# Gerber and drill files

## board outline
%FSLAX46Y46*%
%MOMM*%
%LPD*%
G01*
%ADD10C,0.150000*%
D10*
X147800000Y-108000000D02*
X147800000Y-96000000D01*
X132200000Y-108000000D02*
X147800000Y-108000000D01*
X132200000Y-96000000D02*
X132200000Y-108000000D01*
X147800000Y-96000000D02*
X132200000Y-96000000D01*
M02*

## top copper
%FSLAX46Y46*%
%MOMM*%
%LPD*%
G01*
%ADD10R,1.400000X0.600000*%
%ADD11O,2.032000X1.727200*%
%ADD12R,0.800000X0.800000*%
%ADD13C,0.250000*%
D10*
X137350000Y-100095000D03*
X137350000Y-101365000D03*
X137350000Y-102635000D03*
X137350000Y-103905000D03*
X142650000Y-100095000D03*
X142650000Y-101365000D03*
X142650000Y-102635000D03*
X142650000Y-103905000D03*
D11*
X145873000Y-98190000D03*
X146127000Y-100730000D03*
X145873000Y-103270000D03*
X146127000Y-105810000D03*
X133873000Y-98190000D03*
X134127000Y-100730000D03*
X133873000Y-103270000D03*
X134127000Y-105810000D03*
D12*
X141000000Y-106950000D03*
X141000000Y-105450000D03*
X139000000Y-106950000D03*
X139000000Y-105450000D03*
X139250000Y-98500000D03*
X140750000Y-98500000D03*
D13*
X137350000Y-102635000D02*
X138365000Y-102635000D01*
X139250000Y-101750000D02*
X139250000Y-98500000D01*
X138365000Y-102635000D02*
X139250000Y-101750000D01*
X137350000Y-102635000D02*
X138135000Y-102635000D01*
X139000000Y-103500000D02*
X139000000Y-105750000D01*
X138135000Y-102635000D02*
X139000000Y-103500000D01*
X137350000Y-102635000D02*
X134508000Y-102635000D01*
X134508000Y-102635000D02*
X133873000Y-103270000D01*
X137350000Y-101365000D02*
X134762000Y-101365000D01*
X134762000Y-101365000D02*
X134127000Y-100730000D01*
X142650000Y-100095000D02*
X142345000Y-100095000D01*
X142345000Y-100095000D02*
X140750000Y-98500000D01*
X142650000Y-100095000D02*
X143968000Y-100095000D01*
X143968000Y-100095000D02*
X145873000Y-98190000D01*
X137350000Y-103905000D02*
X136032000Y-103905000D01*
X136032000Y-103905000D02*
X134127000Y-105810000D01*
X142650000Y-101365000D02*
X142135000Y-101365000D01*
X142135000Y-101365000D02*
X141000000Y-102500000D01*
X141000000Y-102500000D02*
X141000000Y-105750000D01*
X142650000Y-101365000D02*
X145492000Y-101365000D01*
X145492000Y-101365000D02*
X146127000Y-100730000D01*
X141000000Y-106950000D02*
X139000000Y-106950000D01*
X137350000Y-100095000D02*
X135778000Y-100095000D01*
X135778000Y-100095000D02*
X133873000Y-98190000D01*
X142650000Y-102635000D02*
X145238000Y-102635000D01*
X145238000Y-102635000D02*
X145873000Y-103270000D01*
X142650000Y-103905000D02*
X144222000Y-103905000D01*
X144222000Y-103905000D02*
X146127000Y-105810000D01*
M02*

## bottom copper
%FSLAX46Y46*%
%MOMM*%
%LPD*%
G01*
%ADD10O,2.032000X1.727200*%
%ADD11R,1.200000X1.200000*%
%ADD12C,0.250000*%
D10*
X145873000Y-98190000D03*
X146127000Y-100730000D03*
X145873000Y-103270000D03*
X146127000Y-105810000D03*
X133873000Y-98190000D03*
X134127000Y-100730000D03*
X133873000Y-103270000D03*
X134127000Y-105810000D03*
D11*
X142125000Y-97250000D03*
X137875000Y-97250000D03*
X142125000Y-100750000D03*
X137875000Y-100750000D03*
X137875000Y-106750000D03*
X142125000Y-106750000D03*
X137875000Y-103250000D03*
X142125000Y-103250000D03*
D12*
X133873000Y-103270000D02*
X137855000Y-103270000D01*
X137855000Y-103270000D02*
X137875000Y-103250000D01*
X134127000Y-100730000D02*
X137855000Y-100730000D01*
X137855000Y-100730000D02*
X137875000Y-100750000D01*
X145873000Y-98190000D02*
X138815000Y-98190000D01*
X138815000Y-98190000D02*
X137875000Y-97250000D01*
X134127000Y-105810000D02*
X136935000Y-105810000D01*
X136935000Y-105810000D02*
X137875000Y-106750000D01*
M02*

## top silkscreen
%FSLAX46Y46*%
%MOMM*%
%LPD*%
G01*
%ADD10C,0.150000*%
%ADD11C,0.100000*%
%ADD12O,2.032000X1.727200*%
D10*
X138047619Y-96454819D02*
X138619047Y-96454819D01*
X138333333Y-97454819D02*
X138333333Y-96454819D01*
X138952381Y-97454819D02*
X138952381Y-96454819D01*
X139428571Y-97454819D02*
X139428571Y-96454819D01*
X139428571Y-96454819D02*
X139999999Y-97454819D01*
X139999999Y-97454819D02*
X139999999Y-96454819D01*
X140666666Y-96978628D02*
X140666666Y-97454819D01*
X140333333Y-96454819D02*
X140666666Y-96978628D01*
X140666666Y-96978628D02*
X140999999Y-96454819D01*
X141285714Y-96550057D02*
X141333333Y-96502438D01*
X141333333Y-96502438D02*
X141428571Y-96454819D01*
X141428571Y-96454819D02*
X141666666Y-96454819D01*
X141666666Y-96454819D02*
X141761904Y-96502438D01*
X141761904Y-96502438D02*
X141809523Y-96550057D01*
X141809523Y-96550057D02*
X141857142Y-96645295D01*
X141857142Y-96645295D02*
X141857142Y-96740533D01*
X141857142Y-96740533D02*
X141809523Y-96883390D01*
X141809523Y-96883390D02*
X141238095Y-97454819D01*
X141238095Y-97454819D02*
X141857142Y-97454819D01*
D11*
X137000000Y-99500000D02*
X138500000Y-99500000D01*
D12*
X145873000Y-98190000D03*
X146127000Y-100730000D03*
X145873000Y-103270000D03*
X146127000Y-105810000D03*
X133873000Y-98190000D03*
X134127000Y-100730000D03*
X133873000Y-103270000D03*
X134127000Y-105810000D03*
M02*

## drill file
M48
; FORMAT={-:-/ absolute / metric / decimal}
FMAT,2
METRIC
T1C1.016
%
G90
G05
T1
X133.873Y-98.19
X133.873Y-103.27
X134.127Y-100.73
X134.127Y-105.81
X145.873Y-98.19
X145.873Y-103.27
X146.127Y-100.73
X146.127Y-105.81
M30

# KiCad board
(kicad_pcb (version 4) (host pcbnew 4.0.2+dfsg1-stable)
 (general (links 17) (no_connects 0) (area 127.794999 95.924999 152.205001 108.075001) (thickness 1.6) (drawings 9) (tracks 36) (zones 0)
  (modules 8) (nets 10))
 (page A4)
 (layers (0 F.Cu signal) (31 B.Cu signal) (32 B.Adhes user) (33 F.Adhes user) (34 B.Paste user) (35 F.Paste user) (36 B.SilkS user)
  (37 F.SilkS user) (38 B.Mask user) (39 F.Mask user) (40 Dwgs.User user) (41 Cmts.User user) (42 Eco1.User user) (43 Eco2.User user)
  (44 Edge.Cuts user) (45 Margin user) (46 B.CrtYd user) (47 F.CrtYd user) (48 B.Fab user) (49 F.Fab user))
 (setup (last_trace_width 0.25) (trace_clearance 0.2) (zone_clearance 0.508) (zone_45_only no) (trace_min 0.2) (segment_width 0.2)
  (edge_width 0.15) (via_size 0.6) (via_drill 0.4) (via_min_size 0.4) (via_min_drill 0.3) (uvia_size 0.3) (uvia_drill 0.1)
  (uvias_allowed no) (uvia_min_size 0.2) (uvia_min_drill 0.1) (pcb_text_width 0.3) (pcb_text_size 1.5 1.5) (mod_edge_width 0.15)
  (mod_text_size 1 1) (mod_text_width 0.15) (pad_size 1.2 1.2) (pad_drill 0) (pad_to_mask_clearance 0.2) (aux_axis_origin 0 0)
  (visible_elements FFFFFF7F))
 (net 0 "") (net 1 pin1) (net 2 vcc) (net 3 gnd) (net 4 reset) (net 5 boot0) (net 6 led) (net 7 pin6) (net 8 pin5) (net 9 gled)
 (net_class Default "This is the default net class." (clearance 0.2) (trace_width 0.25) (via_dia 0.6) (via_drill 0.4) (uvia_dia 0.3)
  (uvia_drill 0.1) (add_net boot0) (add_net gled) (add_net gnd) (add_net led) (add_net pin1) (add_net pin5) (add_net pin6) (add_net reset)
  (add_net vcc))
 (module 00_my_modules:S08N (layer F.Cu) (at 140 102)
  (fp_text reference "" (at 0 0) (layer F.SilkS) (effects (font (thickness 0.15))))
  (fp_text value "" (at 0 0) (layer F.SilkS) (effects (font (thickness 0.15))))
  (fp_line (start -3 -2.5) (end -1.5 -2.5) (layer F.SilkS) (width 0.1))
  (pad 1 smd rect (at -2.65 -1.905) (size 1.4 0.6) (layers F.Cu F.Paste F.Mask) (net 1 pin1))
  (pad VCC smd rect (at -2.65 -0.635) (size 1.4 0.6) (layers F.Cu F.Paste F.Mask) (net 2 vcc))
  (pad GND smd rect (at -2.65 0.635) (size 1.4 0.6) (layers F.Cu F.Paste F.Mask) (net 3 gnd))
  (pad NRST smd rect (at -2.65 1.905) (size 1.4 0.6) (layers F.Cu F.Paste F.Mask) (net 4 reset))
  (pad BOOT smd rect (at 2.65 -1.905) (size 1.4 0.6) (layers F.Cu F.Paste F.Mask) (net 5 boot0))
  (pad PA13 smd rect (at 2.65 -0.635) (size 1.4 0.6) (layers F.Cu F.Paste F.Mask) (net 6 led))
  (pad 6 smd rect (at 2.65 0.635) (size 1.4 0.6) (layers F.Cu F.Paste F.Mask) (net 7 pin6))
  (pad 5 smd rect (at 2.65 1.905) (size 1.4 0.6) (layers F.Cu F.Paste F.Mask) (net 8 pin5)))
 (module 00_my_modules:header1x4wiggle (layer F.Cu) (at 146 102)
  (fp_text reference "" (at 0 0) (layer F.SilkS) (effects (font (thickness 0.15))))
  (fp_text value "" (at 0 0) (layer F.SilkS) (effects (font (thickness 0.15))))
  (pad BOOT thru_hole oval (at -0.127 -3.81) (size 2.032 1.7272) (drill 1.016) (layers *.Cu *.Mask F.SilkS) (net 5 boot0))
  (pad LED thru_hole oval (at 0.127 -1.27) (size 2.032 1.7272) (drill 1.016) (layers *.Cu *.Mask F.SilkS) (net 6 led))
  (pad 6 thru_hole oval (at -0.127 1.27) (size 2.032 1.7272) (drill 1.016) (layers *.Cu *.Mask F.SilkS) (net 7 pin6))
  (pad 5 thru_hole oval (at 0.127 3.81) (size 2.032 1.7272) (drill 1.016) (layers *.Cu *.Mask F.SilkS) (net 8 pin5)))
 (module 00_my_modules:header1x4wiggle (layer F.Cu) (at 134 102)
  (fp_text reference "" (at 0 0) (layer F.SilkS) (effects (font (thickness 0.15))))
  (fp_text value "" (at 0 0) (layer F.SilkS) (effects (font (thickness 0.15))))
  (pad 1 thru_hole oval (at -0.127 -3.81) (size 2.032 1.7272) (drill 1.016) (layers *.Cu *.Mask F.SilkS) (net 1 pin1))
  (pad VCC thru_hole oval (at 0.127 -1.27) (size 2.032 1.7272) (drill 1.016) (layers *.Cu *.Mask F.SilkS) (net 2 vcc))
  (pad GND thru_hole oval (at -0.127 1.27) (size 2.032 1.7272) (drill 1.016) (layers *.Cu *.Mask F.SilkS) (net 3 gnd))
  (pad NRST thru_hole oval (at 0.127 3.81) (size 2.032 1.7272) (drill 1.016) (layers *.Cu *.Mask F.SilkS) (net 4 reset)))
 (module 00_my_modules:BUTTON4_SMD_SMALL (layer B.Cu) (at 140 99 180)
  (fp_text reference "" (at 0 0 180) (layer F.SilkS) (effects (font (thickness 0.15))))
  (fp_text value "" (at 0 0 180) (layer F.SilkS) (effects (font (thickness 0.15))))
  (pad 1 smd rect (at -2.125 1.75 180) (size 1.2 1.2) (layers B.Cu B.Paste B.Mask))
  (pad 2 smd rect (at 2.125 1.75 180) (size 1.2 1.2) (layers B.Cu B.Paste B.Mask) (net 5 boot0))
  (pad 3 smd rect (at -2.125 -1.75 180) (size 1.2 1.2) (layers B.Cu B.Paste B.Mask))
  (pad 4 smd rect (at 2.125 -1.75 180) (size 1.2 1.2) (layers B.Cu B.Paste B.Mask) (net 2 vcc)))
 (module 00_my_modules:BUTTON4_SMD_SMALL (layer B.Cu) (at 140 105)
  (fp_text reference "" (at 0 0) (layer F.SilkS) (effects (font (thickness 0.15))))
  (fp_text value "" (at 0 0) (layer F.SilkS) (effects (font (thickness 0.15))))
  (pad 1 smd rect (at -2.125 1.75) (size 1.2 1.2) (layers B.Cu B.Paste B.Mask) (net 4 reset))
  (pad 2 smd rect (at 2.125 1.75) (size 1.2 1.2) (layers B.Cu B.Paste B.Mask))
  (pad 3 smd rect (at -2.125 -1.75) (size 1.2 1.2) (layers B.Cu B.Paste B.Mask) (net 3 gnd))
  (pad 4 smd rect (at 2.125 -1.75) (size 1.2 1.2) (layers B.Cu B.Paste B.Mask)))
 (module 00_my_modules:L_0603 (layer F.Cu) (at 141 106.2 90)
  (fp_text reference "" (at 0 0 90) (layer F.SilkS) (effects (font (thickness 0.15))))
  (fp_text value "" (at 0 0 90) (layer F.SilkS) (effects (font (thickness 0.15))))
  (pad 1 smd rect (at -0.75 0 90) (size 0.8 0.8) (layers F.Cu F.Paste F.Mask) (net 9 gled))
  (pad 2 smd rect (at 0.75 0 90) (size 0.8 0.8) (layers F.Cu F.Paste F.Mask) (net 6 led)))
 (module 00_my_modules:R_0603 (layer F.Cu) (at 139 106.2 90)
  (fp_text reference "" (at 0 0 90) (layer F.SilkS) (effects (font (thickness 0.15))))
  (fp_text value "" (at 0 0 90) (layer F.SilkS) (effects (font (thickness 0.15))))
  (pad 1 smd rect (at -0.75 0 90) (size 0.8 0.8) (layers F.Cu F.Paste F.Mask) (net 9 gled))
  (pad 2 smd rect (at 0.75 0 90) (size 0.8 0.8) (layers F.Cu F.Paste F.Mask) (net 3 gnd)))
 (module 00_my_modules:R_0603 (layer F.Cu) (at 140 98.5)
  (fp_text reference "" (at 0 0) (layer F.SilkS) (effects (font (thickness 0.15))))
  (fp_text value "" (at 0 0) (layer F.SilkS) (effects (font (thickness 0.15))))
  (pad 1 smd rect (at -0.75 0) (size 0.8 0.8) (layers F.Cu F.Paste F.Mask) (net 3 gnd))
  (pad 2 smd rect (at 0.75 0) (size 0.8 0.8) (layers F.Cu F.Paste F.Mask) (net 5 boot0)))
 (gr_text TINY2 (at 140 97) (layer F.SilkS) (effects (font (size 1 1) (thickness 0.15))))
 (gr_line (start 147.8 108) (end 147.8 96) (angle 90) (layer Edge.Cuts) (width 0.15))
 (gr_line (start 132.2 108) (end 147.8 108) (angle 90) (layer Edge.Cuts) (width 0.15))
 (gr_line (start 132.2 96) (end 132.2 108) (angle 90) (layer Edge.Cuts) (width 0.15))
 (gr_line (start 147.8 96) (end 132.2 96) (angle 90) (layer Edge.Cuts) (width 0.15))
 (segment (start 137.35 102.635) (end 138.365 102.635) (width 0.25) (layer F.Cu) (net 3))
 (segment (start 139.25 101.75) (end 139.25 98.5) (width 0.25) (layer F.Cu) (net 3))
 (segment (start 138.365 102.635) (end 139.25 101.75) (width 0.25) (layer F.Cu) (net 3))
 (segment (start 137.35 102.635) (end 138.135 102.635) (width 0.25) (layer F.Cu) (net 3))
 (segment (start 139 103.5) (end 139 105.75) (width 0.25) (layer F.Cu) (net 3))
 (segment (start 138.135 102.635) (end 139 103.5) (width 0.25) (layer F.Cu) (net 3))
 (segment (start 133.873 103.27) (end 137.855 103.27) (width 0.25) (layer B.Cu) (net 3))
 (segment (start 137.855 103.27) (end 137.875 103.25) (width 0.25) (layer B.Cu) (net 3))
 (segment (start 137.35 102.635) (end 134.508 102.635) (width 0.25) (layer F.Cu) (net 3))
 (segment (start 134.508 102.635) (end 133.873 103.27) (width 0.25) (layer F.Cu) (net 3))
 (segment (start 134.127 100.73) (end 137.855 100.73) (width 0.25) (layer B.Cu) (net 2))
 (segment (start 137.855 100.73) (end 137.875 100.75) (width 0.25) (layer B.Cu) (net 2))
 (segment (start 137.35 101.365) (end 134.762 101.365) (width 0.25) (layer F.Cu) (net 2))
 (segment (start 134.762 101.365) (end 134.127 100.73) (width 0.25) (layer F.Cu) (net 2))
 (segment (start 145.873 98.19) (end 138.815 98.19) (width 0.25) (layer B.Cu) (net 5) (status 400000))
 (segment (start 138.815 98.19) (end 137.875 97.25) (width 0.25) (layer B.Cu) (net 5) (status 800000))
 (segment (start 142.65 100.095) (end 142.345 100.095) (width 0.25) (layer F.Cu) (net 5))
 (segment (start 142.345 100.095) (end 140.75 98.5) (width 0.25) (layer F.Cu) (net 5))
 (segment (start 142.65 100.095) (end 143.968 100.095) (width 0.25) (layer F.Cu) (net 5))
 (segment (start 143.968 100.095) (end 145.873 98.19) (width 0.25) (layer F.Cu) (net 5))
 (segment (start 134.127 105.81) (end 136.935 105.81) (width 0.25) (layer B.Cu) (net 4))
 (segment (start 136.935 105.81) (end 137.875 106.75) (width 0.25) (layer B.Cu) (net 4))
 (segment (start 137.35 103.905) (end 136.032 103.905) (width 0.25) (layer F.Cu) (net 4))
 (segment (start 136.032 103.905) (end 134.127 105.81) (width 0.25) (layer F.Cu) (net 4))
 (segment (start 142.65 101.365) (end 142.135 101.365) (width 0.25) (layer F.Cu) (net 6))
 (segment (start 142.135 101.365) (end 141 102.5) (width 0.25) (layer F.Cu) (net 6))
 (segment (start 141 102.5) (end 141 105.75) (width 0.25) (layer F.Cu) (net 6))
 (segment (start 142.65 101.365) (end 145.492 101.365) (width 0.25) (layer F.Cu) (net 6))
 (segment (start 145.492 101.365) (end 146.127 100.73) (width 0.25) (layer F.Cu) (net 6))
 (segment (start 141 106.95) (end 139 106.95) (width 0.25) (layer F.Cu) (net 9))
 (segment (start 137.35 100.095) (end 135.778 100.095) (width 0.25) (layer F.Cu) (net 1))
 (segment (start 135.778 100.095) (end 133.873 98.19) (width 0.25) (layer F.Cu) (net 1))
 (segment (start 142.65 102.635) (end 145.238 102.635) (width 0.25) (layer F.Cu) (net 7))
 (segment (start 145.238 102.635) (end 145.873 103.27) (width 0.25) (layer F.Cu) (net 7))
 (segment (start 142.65 103.905) (end 144.222 103.905) (width 0.25) (layer F.Cu) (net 8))
 (segment (start 144.222 103.905) (end 146.127 105.81) (width 0.25) (layer F.Cu) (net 8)))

